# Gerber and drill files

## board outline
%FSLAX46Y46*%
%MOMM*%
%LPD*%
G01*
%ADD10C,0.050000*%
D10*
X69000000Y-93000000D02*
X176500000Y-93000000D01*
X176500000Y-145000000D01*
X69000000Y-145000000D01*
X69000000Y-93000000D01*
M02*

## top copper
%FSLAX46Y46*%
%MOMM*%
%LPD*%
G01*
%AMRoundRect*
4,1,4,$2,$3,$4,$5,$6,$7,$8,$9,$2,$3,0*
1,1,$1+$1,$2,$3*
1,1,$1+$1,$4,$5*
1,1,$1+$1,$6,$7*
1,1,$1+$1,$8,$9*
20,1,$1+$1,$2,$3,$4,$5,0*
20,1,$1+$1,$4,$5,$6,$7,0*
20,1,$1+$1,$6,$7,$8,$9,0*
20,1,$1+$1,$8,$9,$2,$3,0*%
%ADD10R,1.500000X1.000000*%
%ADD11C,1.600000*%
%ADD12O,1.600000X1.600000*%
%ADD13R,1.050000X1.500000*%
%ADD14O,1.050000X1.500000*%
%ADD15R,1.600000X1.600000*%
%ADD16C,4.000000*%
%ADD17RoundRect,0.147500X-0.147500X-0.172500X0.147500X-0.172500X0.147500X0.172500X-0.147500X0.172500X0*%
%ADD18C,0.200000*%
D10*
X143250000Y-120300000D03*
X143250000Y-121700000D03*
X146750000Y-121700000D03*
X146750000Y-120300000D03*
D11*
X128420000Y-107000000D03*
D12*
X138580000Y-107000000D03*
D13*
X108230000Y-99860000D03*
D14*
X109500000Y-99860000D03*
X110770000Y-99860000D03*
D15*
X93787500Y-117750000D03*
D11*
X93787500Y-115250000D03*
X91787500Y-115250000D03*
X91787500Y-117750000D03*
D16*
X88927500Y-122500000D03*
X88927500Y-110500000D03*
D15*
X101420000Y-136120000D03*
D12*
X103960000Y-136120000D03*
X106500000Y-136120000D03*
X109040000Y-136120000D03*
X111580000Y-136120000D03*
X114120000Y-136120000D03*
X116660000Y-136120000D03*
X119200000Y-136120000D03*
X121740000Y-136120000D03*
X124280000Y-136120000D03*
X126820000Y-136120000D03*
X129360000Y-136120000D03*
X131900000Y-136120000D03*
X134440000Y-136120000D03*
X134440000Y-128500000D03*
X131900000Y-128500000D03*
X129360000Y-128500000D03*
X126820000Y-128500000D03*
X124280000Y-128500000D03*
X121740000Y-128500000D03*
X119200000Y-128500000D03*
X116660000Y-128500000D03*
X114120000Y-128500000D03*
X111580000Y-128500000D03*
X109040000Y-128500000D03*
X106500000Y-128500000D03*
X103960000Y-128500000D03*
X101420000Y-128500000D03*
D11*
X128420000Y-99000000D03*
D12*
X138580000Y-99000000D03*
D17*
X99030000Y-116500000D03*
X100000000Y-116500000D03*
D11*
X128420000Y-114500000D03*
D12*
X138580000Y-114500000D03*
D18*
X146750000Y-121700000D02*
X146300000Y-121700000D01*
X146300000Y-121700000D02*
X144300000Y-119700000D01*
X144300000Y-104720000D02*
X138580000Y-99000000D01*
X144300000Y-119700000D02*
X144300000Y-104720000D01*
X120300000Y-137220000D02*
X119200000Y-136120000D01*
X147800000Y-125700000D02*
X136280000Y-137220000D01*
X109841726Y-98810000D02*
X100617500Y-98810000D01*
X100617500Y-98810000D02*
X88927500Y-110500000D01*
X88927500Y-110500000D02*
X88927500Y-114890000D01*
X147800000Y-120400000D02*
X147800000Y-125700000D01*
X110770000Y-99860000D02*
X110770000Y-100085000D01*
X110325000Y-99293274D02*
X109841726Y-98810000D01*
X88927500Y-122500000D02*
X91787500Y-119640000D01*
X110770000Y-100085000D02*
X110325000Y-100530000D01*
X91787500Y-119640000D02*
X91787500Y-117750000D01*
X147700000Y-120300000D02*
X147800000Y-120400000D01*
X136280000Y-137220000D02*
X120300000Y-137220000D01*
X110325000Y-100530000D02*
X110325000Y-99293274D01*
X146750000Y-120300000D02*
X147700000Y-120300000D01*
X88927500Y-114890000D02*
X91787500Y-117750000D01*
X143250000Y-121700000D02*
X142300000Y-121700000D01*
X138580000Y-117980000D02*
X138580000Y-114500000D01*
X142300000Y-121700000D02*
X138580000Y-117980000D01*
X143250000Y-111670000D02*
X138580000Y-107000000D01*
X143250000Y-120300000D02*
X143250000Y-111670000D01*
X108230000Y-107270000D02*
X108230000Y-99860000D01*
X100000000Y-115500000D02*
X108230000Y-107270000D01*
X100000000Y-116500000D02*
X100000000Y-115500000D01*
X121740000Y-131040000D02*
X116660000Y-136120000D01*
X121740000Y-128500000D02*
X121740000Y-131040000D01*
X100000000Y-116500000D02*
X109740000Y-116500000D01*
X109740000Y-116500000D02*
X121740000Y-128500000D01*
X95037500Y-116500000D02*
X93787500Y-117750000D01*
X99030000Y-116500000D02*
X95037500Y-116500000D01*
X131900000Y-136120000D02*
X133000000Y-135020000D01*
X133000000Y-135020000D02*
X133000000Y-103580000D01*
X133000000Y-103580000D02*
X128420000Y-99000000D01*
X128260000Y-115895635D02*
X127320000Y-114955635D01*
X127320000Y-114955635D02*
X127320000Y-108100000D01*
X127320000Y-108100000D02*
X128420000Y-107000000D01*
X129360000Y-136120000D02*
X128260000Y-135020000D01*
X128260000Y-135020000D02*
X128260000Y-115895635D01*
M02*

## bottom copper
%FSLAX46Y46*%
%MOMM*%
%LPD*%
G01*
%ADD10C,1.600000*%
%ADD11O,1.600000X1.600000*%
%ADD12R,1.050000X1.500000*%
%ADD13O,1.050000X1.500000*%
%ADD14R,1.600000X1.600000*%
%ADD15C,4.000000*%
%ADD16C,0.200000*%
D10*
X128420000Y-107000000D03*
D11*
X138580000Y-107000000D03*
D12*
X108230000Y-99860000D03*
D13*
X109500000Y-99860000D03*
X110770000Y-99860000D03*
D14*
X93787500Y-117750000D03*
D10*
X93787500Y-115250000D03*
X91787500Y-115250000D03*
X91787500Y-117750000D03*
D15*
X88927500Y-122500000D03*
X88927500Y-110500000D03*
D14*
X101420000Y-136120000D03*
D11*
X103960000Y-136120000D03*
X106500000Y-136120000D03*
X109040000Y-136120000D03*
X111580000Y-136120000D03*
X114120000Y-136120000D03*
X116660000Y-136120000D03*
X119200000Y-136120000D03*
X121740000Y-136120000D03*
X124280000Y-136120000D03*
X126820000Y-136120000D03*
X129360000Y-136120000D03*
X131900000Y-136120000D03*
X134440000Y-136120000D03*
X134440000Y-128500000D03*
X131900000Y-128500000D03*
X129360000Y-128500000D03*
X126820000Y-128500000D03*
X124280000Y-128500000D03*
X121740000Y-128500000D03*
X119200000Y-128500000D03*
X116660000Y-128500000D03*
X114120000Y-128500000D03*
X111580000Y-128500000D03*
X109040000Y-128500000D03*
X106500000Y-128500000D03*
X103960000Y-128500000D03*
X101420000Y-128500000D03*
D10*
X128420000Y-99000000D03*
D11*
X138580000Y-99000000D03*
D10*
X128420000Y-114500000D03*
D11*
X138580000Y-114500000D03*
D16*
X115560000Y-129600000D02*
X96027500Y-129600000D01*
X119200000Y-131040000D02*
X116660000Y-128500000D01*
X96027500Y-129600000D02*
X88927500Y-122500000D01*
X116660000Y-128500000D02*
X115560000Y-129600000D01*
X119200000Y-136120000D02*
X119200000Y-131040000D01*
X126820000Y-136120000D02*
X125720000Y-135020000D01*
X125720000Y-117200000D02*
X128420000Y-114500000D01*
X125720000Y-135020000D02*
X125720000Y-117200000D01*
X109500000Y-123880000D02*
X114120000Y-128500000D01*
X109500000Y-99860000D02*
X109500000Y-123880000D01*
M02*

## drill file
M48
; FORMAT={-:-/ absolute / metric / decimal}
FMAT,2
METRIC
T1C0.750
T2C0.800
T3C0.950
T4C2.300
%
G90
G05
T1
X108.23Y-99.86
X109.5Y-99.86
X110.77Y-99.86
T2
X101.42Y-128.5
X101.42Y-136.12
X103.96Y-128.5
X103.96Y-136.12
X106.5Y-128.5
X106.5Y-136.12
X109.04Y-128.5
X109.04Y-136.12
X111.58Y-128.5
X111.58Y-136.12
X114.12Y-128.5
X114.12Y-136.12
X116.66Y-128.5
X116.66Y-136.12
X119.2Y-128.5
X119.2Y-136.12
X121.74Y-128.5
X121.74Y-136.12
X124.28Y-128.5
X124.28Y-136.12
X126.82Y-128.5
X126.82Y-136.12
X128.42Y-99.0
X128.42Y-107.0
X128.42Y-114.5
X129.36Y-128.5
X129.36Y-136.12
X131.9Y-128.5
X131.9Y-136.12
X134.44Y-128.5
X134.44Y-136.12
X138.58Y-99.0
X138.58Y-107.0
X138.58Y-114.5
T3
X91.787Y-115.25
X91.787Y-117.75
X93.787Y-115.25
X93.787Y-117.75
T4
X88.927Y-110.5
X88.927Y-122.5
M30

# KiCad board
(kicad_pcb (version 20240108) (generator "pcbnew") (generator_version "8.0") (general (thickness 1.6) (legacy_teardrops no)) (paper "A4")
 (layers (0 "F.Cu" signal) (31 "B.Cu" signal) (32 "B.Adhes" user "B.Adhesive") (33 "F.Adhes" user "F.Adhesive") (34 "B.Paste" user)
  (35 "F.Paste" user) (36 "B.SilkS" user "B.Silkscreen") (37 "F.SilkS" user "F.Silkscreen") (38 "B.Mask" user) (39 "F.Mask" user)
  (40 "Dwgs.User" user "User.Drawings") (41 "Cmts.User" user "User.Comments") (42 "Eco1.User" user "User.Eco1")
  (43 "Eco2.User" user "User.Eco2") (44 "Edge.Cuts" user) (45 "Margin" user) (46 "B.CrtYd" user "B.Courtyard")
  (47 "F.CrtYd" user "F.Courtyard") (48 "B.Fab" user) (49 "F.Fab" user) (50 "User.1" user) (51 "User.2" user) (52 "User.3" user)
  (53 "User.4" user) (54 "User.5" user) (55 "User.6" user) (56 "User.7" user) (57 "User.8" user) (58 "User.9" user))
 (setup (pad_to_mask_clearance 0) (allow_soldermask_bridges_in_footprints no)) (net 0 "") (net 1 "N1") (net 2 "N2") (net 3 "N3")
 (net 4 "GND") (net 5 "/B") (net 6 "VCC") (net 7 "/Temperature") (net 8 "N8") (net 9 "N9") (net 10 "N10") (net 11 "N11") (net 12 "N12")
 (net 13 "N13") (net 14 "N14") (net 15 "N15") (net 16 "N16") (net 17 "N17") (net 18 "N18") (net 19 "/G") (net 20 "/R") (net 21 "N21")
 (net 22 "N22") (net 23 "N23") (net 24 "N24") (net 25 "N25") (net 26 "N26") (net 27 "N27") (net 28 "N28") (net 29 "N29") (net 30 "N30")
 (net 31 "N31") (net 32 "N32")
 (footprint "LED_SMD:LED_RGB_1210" (layer "F.Cu") (at 145 121)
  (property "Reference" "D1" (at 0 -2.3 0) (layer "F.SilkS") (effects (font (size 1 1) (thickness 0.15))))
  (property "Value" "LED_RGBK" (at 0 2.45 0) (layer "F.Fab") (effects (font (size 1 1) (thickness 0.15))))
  (pad "1" smd rect (at -1.75 -0.7 180) (size 1.5 1) (layers "F.Cu" "F.Paste" "F.Mask") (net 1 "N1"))
  (pad "2" smd rect (at -1.75 0.7 180) (size 1.5 1) (layers "F.Cu" "F.Paste" "F.Mask") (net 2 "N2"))
  (pad "3" smd rect (at 1.75 0.7 180) (size 1.5 1) (layers "F.Cu" "F.Paste" "F.Mask") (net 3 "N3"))
  (pad "4" smd rect (at 1.75 -0.7 180) (size 1.5 1) (layers "F.Cu" "F.Paste" "F.Mask") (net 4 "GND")))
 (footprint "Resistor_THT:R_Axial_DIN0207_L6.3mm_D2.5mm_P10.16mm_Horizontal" (layer "F.Cu") (at 128.42 107)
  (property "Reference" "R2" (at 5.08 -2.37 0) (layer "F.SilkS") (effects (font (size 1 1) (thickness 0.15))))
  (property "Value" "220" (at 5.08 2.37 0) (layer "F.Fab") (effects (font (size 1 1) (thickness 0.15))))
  (pad "1" thru_hole circle (at 0 0) (size 1.6 1.6) (drill 0.8) (layers "*.Cu" "*.Mask") (remove_unused_layers no) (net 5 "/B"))
  (pad "2" thru_hole oval (at 10.16 0) (size 1.6 1.6) (drill 0.8) (layers "*.Cu" "*.Mask") (remove_unused_layers no) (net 1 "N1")))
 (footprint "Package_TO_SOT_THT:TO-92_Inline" (layer "F.Cu") (at 108.23 99.86)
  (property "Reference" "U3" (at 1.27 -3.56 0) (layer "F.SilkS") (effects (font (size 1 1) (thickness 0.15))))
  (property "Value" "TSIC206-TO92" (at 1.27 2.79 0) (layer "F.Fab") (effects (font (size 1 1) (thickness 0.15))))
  (pad "1" thru_hole rect (at 0 0) (size 1.05 1.5) (drill 0.75) (layers "*.Cu" "*.Mask") (remove_unused_layers no) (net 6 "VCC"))
  (pad "2" thru_hole oval (at 1.27 0) (size 1.05 1.5) (drill 0.75) (layers "*.Cu" "*.Mask") (remove_unused_layers no) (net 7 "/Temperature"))
  (pad "3" thru_hole oval (at 2.54 0) (size 1.05 1.5) (drill 0.75) (layers "*.Cu" "*.Mask") (remove_unused_layers no) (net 4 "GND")))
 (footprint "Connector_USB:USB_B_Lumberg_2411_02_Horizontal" (layer "F.Cu") (at 93.7875 117.75 180)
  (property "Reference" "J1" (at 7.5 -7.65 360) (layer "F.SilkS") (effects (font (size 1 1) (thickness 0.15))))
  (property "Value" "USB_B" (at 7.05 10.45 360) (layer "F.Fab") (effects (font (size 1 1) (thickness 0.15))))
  (pad "1" thru_hole rect (at 0 0 270) (size 1.6 1.6) (drill 0.95) (layers "*.Cu" "*.Mask") (remove_unused_layers no) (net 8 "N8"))
  (pad "2" thru_hole circle (at 0 2.5 270) (size 1.6 1.6) (drill 0.95) (layers "*.Cu" "*.Mask") (remove_unused_layers no) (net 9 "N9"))
  (pad "3" thru_hole circle (at 2 2.5 270) (size 1.6 1.6) (drill 0.95) (layers "*.Cu" "*.Mask") (remove_unused_layers no) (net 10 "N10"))
  (pad "4" thru_hole circle (at 2 0 270) (size 1.6 1.6) (drill 0.95) (layers "*.Cu" "*.Mask") (remove_unused_layers no) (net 4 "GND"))
  (pad "5" thru_hole circle (at 4.86 -4.75 270) (size 4 4) (drill 2.3) (layers "*.Cu" "*.Mask") (remove_unused_layers no) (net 4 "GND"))
  (pad "5" thru_hole circle (at 4.86 7.25 270) (size 4 4) (drill 2.3) (layers "*.Cu" "*.Mask") (remove_unused_layers no) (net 4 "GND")))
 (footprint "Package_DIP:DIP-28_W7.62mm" (layer "F.Cu") (at 101.42 136.12 90)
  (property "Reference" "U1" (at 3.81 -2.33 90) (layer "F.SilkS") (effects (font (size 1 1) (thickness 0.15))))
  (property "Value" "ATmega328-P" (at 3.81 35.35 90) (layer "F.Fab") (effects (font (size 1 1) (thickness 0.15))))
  (pad "1" thru_hole rect (at 0 0 90) (size 1.6 1.6) (drill 0.8) (layers "*.Cu" "*.Mask") (remove_unused_layers no) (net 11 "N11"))
  (pad "2" thru_hole oval (at 0 2.54 90) (size 1.6 1.6) (drill 0.8) (layers "*.Cu" "*.Mask") (remove_unused_layers no) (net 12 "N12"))
  (pad "3" thru_hole oval (at 0 5.08 90) (size 1.6 1.6) (drill 0.8) (layers "*.Cu" "*.Mask") (remove_unused_layers no) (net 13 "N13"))
  (pad "4" thru_hole oval (at 0 7.62 90) (size 1.6 1.6) (drill 0.8) (layers "*.Cu" "*.Mask") (remove_unused_layers no) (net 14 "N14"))
  (pad "5" thru_hole oval (at 0 10.16 90) (size 1.6 1.6) (drill 0.8) (layers "*.Cu" "*.Mask") (remove_unused_layers no) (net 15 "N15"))
  (pad "6" thru_hole oval (at 0 12.7 90) (size 1.6 1.6) (drill 0.8) (layers "*.Cu" "*.Mask") (remove_unused_layers no) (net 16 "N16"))
  (pad "7" thru_hole oval (at 0 15.24 90) (size 1.6 1.6) (drill 0.8) (layers "*.Cu" "*.Mask") (remove_unused_layers no) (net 6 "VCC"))
  (pad "8" thru_hole oval (at 0 17.78 90) (size 1.6 1.6) (drill 0.8) (layers "*.Cu" "*.Mask") (remove_unused_layers no) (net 4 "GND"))
  (pad "9" thru_hole oval (at 0 20.32 90) (size 1.6 1.6) (drill 0.8) (layers "*.Cu" "*.Mask") (remove_unused_layers no) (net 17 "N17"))
  (pad "10" thru_hole oval (at 0 22.86 90) (size 1.6 1.6) (drill 0.8) (layers "*.Cu" "*.Mask") (remove_unused_layers no) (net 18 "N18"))
  (pad "11" thru_hole oval (at 0 25.4 90) (size 1.6 1.6) (drill 0.8) (layers "*.Cu" "*.Mask") (remove_unused_layers no) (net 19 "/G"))
  (pad "12" thru_hole oval (at 0 27.94 90) (size 1.6 1.6) (drill 0.8) (layers "*.Cu" "*.Mask") (remove_unused_layers no) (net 5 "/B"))
  (pad "13" thru_hole oval (at 0 30.48 90) (size 1.6 1.6) (drill 0.8) (layers "*.Cu" "*.Mask") (remove_unused_layers no) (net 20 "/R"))
  (pad "14" thru_hole oval (at 0 33.02 90) (size 1.6 1.6) (drill 0.8) (layers "*.Cu" "*.Mask") (remove_unused_layers no) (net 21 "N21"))
  (pad "15" thru_hole oval (at 7.62 33.02 90) (size 1.6 1.6) (drill 0.8) (layers "*.Cu" "*.Mask") (remove_unused_layers no) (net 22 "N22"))
  (pad "16" thru_hole oval (at 7.62 30.48 90) (size 1.6 1.6) (drill 0.8) (layers "*.Cu" "*.Mask") (remove_unused_layers no) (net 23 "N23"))
  (pad "17" thru_hole oval (at 7.62 27.94 90) (size 1.6 1.6) (drill 0.8) (layers "*.Cu" "*.Mask") (remove_unused_layers no) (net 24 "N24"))
  (pad "18" thru_hole oval (at 7.62 25.4 90) (size 1.6 1.6) (drill 0.8) (layers "*.Cu" "*.Mask") (remove_unused_layers no) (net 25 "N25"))
  (pad "19" thru_hole oval (at 7.62 22.86 90) (size 1.6 1.6) (drill 0.8) (layers "*.Cu" "*.Mask") (remove_unused_layers no) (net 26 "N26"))
  (pad "20" thru_hole oval (at 7.62 20.32 90) (size 1.6 1.6) (drill 0.8) (layers "*.Cu" "*.Mask") (remove_unused_layers no) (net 6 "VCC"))
  (pad "21" thru_hole oval (at 7.62 17.78 90) (size 1.6 1.6) (drill 0.8) (layers "*.Cu" "*.Mask") (remove_unused_layers no) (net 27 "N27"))
  (pad "22" thru_hole oval (at 7.62 15.24 90) (size 1.6 1.6) (drill 0.8) (layers "*.Cu" "*.Mask") (remove_unused_layers no) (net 4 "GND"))
  (pad "23" thru_hole oval (at 7.62 12.7 90) (size 1.6 1.6) (drill 0.8) (layers "*.Cu" "*.Mask") (remove_unused_layers no)
   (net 7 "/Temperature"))
  (pad "24" thru_hole oval (at 7.62 10.16 90) (size 1.6 1.6) (drill 0.8) (layers "*.Cu" "*.Mask") (remove_unused_layers no) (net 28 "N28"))
  (pad "25" thru_hole oval (at 7.62 7.62 90) (size 1.6 1.6) (drill 0.8) (layers "*.Cu" "*.Mask") (remove_unused_layers no) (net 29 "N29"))
  (pad "26" thru_hole oval (at 7.62 5.08 90) (size 1.6 1.6) (drill 0.8) (layers "*.Cu" "*.Mask") (remove_unused_layers no) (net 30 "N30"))
  (pad "27" thru_hole oval (at 7.62 2.54 90) (size 1.6 1.6) (drill 0.8) (layers "*.Cu" "*.Mask") (remove_unused_layers no) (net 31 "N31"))
  (pad "28" thru_hole oval (at 7.62 0 90) (size 1.6 1.6) (drill 0.8) (layers "*.Cu" "*.Mask") (remove_unused_layers no) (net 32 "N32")))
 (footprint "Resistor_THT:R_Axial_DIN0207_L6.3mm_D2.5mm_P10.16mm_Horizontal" (layer "F.Cu") (at 128.42 99)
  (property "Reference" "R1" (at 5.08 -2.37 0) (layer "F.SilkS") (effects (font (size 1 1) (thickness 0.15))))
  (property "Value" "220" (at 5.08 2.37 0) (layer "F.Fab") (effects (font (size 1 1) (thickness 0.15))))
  (pad "1" thru_hole circle (at 0 0) (size 1.6 1.6) (drill 0.8) (layers "*.Cu" "*.Mask") (remove_unused_layers no) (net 20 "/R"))
  (pad "2" thru_hole oval (at 10.16 0) (size 1.6 1.6) (drill 0.8) (layers "*.Cu" "*.Mask") (remove_unused_layers no) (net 3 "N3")))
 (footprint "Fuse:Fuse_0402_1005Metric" (layer "F.Cu") (at 99.515 116.5)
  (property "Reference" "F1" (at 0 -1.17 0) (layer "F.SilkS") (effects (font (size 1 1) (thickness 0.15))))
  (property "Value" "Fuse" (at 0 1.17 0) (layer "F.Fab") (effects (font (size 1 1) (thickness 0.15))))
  (pad "1" smd roundrect (at -0.485 0) (size 0.59 0.64) (layers "F.Cu" "F.Paste" "F.Mask") (roundrect_rratio 0.25) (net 8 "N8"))
  (pad "2" smd roundrect (at 0.485 0) (size 0.59 0.64) (layers "F.Cu" "F.Paste" "F.Mask") (roundrect_rratio 0.25) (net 6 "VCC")))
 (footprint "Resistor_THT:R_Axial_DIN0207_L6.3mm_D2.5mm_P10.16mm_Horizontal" (layer "F.Cu") (at 128.42 114.5)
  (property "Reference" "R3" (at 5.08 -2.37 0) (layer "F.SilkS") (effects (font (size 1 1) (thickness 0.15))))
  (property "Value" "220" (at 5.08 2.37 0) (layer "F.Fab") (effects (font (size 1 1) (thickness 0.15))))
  (pad "1" thru_hole circle (at 0 0) (size 1.6 1.6) (drill 0.8) (layers "*.Cu" "*.Mask") (remove_unused_layers no) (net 19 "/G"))
  (pad "2" thru_hole oval (at 10.16 0) (size 1.6 1.6) (drill 0.8) (layers "*.Cu" "*.Mask") (remove_unused_layers no) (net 2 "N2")))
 (gr_rect (start 69 93) (end 176.5 145) (stroke (width 0.05) (type default)) (fill none) (layer "Edge.Cuts"))
 (segment (start 146.75 121.7) (end 146.3 121.7) (width 0.2) (layer "F.Cu") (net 3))
 (segment (start 146.3 121.7) (end 144.3 119.7) (width 0.2) (layer "F.Cu") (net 3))
 (segment (start 144.3 104.72) (end 138.58 99) (width 0.2) (layer "F.Cu") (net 3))
 (segment (start 144.3 119.7) (end 144.3 104.72) (width 0.2) (layer "F.Cu") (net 3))
 (segment (start 120.3 137.22) (end 119.2 136.12) (width 0.2) (layer "F.Cu") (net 4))
 (segment (start 147.8 125.7) (end 136.28 137.22) (width 0.2) (layer "F.Cu") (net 4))
 (segment (start 109.841726 98.81) (end 100.6175 98.81) (width 0.2) (layer "F.Cu") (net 4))
 (segment (start 100.6175 98.81) (end 88.9275 110.5) (width 0.2) (layer "F.Cu") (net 4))
 (segment (start 88.9275 110.5) (end 88.9275 114.89) (width 0.2) (layer "F.Cu") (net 4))
 (segment (start 147.8 120.4) (end 147.8 125.7) (width 0.2) (layer "F.Cu") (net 4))
 (segment (start 110.77 99.86) (end 110.77 100.085) (width 0.2) (layer "F.Cu") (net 4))
 (segment (start 110.325 99.293274) (end 109.841726 98.81) (width 0.2) (layer "F.Cu") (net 4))
 (segment (start 88.9275 122.5) (end 91.7875 119.64) (width 0.2) (layer "F.Cu") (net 4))
 (segment (start 110.77 100.085) (end 110.325 100.53) (width 0.2) (layer "F.Cu") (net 4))
 (segment (start 91.7875 119.64) (end 91.7875 117.75) (width 0.2) (layer "F.Cu") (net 4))
 (segment (start 147.7 120.3) (end 147.8 120.4) (width 0.2) (layer "F.Cu") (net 4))
 (segment (start 136.28 137.22) (end 120.3 137.22) (width 0.2) (layer "F.Cu") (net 4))
 (segment (start 110.325 100.53) (end 110.325 99.293274) (width 0.2) (layer "F.Cu") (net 4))
 (segment (start 146.75 120.3) (end 147.7 120.3) (width 0.2) (layer "F.Cu") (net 4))
 (segment (start 88.9275 114.89) (end 91.7875 117.75) (width 0.2) (layer "F.Cu") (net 4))
 (segment (start 115.56 129.6) (end 96.0275 129.6) (width 0.2) (layer "B.Cu") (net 4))
 (segment (start 119.2 131.04) (end 116.66 128.5) (width 0.2) (layer "B.Cu") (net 4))
 (segment (start 96.0275 129.6) (end 88.9275 122.5) (width 0.2) (layer "B.Cu") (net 4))
 (segment (start 116.66 128.5) (end 115.56 129.6) (width 0.2) (layer "B.Cu") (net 4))
 (segment (start 119.2 136.12) (end 119.2 131.04) (width 0.2) (layer "B.Cu") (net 4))
 (segment (start 143.25 121.7) (end 142.3 121.7) (width 0.2) (layer "F.Cu") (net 2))
 (segment (start 138.58 117.98) (end 138.58 114.5) (width 0.2) (layer "F.Cu") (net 2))
 (segment (start 142.3 121.7) (end 138.58 117.98) (width 0.2) (layer "F.Cu") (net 2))
 (segment (start 143.25 111.67) (end 138.58 107) (width 0.2) (layer "F.Cu") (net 1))
 (segment (start 143.25 120.3) (end 143.25 111.67) (width 0.2) (layer "F.Cu") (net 1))
 (segment (start 108.23 107.27) (end 108.23 99.86) (width 0.2) (layer "F.Cu") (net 6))
 (segment (start 100 115.5) (end 108.23 107.27) (width 0.2) (layer "F.Cu") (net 6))
 (segment (start 100 116.5) (end 100 115.5) (width 0.2) (layer "F.Cu") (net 6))
 (segment (start 121.74 131.04) (end 116.66 136.12) (width 0.2) (layer "F.Cu") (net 6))
 (segment (start 121.74 128.5) (end 121.74 131.04) (width 0.2) (layer "F.Cu") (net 6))
 (segment (start 100 116.5) (end 109.74 116.5) (width 0.2) (layer "F.Cu") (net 6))
 (segment (start 109.74 116.5) (end 121.74 128.5) (width 0.2) (layer "F.Cu") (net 6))
 (segment (start 95.0375 116.5) (end 93.7875 117.75) (width 0.2) (layer "F.Cu") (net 8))
 (segment (start 99.03 116.5) (end 95.0375 116.5) (width 0.2) (layer "F.Cu") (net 8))
 (segment (start 131.9 136.12) (end 133 135.02) (width 0.2) (layer "F.Cu") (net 20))
 (segment (start 133 135.02) (end 133 103.58) (width 0.2) (layer "F.Cu") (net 20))
 (segment (start 133 103.58) (end 128.42 99) (width 0.2) (layer "F.Cu") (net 20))
 (segment (start 128.26 115.895635) (end 127.32 114.955635) (width 0.2) (layer "F.Cu") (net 5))
 (segment (start 127.32 114.955635) (end 127.32 108.1) (width 0.2) (layer "F.Cu") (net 5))
 (segment (start 127.32 108.1) (end 128.42 107) (width 0.2) (layer "F.Cu") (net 5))
 (segment (start 129.36 136.12) (end 128.26 135.02) (width 0.2) (layer "F.Cu") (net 5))
 (segment (start 128.26 135.02) (end 128.26 115.895635) (width 0.2) (layer "F.Cu") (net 5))
 (segment (start 126.82 136.12) (end 125.72 135.02) (width 0.2) (layer "B.Cu") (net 19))
 (segment (start 125.72 117.2) (end 128.42 114.5) (width 0.2) (layer "B.Cu") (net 19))
 (segment (start 125.72 135.02) (end 125.72 117.2) (width 0.2) (layer "B.Cu") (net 19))
 (segment (start 109.5 123.88) (end 114.12 128.5) (width 0.2) (layer "B.Cu") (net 7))
 (segment (start 109.5 99.86) (end 109.5 123.88) (width 0.2) (layer "B.Cu") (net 7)))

